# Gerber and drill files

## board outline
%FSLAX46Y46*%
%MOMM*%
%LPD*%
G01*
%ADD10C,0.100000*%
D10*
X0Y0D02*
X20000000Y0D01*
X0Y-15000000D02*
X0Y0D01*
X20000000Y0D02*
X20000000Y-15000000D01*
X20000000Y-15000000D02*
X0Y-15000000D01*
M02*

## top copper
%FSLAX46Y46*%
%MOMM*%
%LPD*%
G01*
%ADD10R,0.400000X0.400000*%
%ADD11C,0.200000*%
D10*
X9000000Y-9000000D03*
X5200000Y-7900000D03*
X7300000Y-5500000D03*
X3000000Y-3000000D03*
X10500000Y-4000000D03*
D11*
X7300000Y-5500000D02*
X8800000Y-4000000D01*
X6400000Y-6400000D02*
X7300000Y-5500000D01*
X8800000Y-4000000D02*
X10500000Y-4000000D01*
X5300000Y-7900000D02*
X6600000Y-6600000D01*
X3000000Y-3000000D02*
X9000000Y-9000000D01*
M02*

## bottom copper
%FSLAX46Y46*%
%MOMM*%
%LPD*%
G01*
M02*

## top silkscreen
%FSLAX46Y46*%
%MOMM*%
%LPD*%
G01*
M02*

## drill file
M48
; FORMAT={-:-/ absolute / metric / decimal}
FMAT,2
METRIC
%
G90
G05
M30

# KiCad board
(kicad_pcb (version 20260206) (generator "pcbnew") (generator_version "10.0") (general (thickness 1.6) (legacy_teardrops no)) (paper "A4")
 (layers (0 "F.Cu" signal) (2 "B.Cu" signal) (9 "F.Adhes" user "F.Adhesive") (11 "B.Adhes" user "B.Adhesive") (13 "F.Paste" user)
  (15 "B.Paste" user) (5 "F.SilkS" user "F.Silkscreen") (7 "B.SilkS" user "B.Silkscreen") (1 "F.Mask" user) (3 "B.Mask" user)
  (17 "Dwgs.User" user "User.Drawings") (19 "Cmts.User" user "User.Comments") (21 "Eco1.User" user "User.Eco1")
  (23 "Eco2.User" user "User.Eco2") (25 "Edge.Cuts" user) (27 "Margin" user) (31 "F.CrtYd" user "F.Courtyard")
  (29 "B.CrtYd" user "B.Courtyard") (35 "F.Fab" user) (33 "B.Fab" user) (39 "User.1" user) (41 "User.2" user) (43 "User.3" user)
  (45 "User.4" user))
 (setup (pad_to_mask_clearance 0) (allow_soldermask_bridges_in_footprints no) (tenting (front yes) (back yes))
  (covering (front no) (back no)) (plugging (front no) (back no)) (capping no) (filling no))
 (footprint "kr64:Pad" (layer "F.Cu") (at 9 9)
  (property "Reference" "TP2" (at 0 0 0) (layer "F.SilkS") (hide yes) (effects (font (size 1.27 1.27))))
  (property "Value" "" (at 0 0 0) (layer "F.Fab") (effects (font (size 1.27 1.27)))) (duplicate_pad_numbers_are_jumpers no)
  (pad "1" smd rect (at 0 0) (size 0.4 0.4) (layers "F.Cu" "F.Mask" "F.Paste") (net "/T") (thermal_bridge_angle 45)))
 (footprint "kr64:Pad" (layer "F.Cu") (at 5.2 7.9)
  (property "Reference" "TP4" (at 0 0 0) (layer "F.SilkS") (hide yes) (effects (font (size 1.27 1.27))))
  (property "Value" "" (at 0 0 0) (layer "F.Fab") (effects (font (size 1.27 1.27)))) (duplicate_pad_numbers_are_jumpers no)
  (pad "1" smd rect (at 0 0) (size 0.4 0.4) (layers "F.Cu" "F.Mask" "F.Paste") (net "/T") (thermal_bridge_angle 45)))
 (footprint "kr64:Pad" (layer "F.Cu") (at 7.3 5.5)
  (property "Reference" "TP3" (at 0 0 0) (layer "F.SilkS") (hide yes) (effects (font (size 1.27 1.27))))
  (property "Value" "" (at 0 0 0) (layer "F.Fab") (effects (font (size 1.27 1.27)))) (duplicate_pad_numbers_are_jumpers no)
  (pad "1" smd rect (at 0 0) (size 0.4 0.4) (layers "F.Cu" "F.Mask" "F.Paste") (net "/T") (thermal_bridge_angle 45)))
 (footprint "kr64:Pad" (layer "F.Cu") (at 3 3)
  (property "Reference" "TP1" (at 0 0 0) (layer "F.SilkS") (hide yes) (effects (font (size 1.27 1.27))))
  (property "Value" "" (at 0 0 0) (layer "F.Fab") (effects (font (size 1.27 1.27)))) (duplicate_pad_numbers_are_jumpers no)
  (pad "1" smd rect (at 0 0) (size 0.4 0.4) (layers "F.Cu" "F.Mask" "F.Paste") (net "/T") (thermal_bridge_angle 45)))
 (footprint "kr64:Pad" (layer "F.Cu") (at 10.5 4)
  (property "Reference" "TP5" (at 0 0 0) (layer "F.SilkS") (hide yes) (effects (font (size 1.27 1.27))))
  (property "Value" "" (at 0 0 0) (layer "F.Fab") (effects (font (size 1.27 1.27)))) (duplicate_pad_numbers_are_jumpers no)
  (pad "1" smd rect (at 0 0) (size 0.4 0.4) (layers "F.Cu" "F.Mask" "F.Paste") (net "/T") (thermal_bridge_angle 45)))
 (gr_line (start 0 0) (end 20 0) (stroke (width 0.1) (type default)) (layer "Edge.Cuts"))
 (gr_line (start 0 15) (end 0 0) (stroke (width 0.1) (type default)) (layer "Edge.Cuts"))
 (gr_line (start 20 0) (end 20 15) (stroke (width 0.1) (type default)) (layer "Edge.Cuts"))
 (gr_line (start 20 15) (end 0 15) (stroke (width 0.1) (type default)) (layer "Edge.Cuts"))
 (segment (start 7.3 5.5) (end 8.8 4) (width 0.2) (layer "F.Cu") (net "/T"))
 (segment (start 6.4 6.4) (end 7.3 5.5) (width 0.2) (layer "F.Cu") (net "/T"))
 (segment (start 8.8 4) (end 10.5 4) (width 0.2) (layer "F.Cu") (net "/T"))
 (segment (start 5.3 7.9) (end 6.6 6.6) (width 0.2) (layer "F.Cu") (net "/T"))
 (segment (start 3 3) (end 9 9) (width 0.2) (layer "F.Cu") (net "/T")))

